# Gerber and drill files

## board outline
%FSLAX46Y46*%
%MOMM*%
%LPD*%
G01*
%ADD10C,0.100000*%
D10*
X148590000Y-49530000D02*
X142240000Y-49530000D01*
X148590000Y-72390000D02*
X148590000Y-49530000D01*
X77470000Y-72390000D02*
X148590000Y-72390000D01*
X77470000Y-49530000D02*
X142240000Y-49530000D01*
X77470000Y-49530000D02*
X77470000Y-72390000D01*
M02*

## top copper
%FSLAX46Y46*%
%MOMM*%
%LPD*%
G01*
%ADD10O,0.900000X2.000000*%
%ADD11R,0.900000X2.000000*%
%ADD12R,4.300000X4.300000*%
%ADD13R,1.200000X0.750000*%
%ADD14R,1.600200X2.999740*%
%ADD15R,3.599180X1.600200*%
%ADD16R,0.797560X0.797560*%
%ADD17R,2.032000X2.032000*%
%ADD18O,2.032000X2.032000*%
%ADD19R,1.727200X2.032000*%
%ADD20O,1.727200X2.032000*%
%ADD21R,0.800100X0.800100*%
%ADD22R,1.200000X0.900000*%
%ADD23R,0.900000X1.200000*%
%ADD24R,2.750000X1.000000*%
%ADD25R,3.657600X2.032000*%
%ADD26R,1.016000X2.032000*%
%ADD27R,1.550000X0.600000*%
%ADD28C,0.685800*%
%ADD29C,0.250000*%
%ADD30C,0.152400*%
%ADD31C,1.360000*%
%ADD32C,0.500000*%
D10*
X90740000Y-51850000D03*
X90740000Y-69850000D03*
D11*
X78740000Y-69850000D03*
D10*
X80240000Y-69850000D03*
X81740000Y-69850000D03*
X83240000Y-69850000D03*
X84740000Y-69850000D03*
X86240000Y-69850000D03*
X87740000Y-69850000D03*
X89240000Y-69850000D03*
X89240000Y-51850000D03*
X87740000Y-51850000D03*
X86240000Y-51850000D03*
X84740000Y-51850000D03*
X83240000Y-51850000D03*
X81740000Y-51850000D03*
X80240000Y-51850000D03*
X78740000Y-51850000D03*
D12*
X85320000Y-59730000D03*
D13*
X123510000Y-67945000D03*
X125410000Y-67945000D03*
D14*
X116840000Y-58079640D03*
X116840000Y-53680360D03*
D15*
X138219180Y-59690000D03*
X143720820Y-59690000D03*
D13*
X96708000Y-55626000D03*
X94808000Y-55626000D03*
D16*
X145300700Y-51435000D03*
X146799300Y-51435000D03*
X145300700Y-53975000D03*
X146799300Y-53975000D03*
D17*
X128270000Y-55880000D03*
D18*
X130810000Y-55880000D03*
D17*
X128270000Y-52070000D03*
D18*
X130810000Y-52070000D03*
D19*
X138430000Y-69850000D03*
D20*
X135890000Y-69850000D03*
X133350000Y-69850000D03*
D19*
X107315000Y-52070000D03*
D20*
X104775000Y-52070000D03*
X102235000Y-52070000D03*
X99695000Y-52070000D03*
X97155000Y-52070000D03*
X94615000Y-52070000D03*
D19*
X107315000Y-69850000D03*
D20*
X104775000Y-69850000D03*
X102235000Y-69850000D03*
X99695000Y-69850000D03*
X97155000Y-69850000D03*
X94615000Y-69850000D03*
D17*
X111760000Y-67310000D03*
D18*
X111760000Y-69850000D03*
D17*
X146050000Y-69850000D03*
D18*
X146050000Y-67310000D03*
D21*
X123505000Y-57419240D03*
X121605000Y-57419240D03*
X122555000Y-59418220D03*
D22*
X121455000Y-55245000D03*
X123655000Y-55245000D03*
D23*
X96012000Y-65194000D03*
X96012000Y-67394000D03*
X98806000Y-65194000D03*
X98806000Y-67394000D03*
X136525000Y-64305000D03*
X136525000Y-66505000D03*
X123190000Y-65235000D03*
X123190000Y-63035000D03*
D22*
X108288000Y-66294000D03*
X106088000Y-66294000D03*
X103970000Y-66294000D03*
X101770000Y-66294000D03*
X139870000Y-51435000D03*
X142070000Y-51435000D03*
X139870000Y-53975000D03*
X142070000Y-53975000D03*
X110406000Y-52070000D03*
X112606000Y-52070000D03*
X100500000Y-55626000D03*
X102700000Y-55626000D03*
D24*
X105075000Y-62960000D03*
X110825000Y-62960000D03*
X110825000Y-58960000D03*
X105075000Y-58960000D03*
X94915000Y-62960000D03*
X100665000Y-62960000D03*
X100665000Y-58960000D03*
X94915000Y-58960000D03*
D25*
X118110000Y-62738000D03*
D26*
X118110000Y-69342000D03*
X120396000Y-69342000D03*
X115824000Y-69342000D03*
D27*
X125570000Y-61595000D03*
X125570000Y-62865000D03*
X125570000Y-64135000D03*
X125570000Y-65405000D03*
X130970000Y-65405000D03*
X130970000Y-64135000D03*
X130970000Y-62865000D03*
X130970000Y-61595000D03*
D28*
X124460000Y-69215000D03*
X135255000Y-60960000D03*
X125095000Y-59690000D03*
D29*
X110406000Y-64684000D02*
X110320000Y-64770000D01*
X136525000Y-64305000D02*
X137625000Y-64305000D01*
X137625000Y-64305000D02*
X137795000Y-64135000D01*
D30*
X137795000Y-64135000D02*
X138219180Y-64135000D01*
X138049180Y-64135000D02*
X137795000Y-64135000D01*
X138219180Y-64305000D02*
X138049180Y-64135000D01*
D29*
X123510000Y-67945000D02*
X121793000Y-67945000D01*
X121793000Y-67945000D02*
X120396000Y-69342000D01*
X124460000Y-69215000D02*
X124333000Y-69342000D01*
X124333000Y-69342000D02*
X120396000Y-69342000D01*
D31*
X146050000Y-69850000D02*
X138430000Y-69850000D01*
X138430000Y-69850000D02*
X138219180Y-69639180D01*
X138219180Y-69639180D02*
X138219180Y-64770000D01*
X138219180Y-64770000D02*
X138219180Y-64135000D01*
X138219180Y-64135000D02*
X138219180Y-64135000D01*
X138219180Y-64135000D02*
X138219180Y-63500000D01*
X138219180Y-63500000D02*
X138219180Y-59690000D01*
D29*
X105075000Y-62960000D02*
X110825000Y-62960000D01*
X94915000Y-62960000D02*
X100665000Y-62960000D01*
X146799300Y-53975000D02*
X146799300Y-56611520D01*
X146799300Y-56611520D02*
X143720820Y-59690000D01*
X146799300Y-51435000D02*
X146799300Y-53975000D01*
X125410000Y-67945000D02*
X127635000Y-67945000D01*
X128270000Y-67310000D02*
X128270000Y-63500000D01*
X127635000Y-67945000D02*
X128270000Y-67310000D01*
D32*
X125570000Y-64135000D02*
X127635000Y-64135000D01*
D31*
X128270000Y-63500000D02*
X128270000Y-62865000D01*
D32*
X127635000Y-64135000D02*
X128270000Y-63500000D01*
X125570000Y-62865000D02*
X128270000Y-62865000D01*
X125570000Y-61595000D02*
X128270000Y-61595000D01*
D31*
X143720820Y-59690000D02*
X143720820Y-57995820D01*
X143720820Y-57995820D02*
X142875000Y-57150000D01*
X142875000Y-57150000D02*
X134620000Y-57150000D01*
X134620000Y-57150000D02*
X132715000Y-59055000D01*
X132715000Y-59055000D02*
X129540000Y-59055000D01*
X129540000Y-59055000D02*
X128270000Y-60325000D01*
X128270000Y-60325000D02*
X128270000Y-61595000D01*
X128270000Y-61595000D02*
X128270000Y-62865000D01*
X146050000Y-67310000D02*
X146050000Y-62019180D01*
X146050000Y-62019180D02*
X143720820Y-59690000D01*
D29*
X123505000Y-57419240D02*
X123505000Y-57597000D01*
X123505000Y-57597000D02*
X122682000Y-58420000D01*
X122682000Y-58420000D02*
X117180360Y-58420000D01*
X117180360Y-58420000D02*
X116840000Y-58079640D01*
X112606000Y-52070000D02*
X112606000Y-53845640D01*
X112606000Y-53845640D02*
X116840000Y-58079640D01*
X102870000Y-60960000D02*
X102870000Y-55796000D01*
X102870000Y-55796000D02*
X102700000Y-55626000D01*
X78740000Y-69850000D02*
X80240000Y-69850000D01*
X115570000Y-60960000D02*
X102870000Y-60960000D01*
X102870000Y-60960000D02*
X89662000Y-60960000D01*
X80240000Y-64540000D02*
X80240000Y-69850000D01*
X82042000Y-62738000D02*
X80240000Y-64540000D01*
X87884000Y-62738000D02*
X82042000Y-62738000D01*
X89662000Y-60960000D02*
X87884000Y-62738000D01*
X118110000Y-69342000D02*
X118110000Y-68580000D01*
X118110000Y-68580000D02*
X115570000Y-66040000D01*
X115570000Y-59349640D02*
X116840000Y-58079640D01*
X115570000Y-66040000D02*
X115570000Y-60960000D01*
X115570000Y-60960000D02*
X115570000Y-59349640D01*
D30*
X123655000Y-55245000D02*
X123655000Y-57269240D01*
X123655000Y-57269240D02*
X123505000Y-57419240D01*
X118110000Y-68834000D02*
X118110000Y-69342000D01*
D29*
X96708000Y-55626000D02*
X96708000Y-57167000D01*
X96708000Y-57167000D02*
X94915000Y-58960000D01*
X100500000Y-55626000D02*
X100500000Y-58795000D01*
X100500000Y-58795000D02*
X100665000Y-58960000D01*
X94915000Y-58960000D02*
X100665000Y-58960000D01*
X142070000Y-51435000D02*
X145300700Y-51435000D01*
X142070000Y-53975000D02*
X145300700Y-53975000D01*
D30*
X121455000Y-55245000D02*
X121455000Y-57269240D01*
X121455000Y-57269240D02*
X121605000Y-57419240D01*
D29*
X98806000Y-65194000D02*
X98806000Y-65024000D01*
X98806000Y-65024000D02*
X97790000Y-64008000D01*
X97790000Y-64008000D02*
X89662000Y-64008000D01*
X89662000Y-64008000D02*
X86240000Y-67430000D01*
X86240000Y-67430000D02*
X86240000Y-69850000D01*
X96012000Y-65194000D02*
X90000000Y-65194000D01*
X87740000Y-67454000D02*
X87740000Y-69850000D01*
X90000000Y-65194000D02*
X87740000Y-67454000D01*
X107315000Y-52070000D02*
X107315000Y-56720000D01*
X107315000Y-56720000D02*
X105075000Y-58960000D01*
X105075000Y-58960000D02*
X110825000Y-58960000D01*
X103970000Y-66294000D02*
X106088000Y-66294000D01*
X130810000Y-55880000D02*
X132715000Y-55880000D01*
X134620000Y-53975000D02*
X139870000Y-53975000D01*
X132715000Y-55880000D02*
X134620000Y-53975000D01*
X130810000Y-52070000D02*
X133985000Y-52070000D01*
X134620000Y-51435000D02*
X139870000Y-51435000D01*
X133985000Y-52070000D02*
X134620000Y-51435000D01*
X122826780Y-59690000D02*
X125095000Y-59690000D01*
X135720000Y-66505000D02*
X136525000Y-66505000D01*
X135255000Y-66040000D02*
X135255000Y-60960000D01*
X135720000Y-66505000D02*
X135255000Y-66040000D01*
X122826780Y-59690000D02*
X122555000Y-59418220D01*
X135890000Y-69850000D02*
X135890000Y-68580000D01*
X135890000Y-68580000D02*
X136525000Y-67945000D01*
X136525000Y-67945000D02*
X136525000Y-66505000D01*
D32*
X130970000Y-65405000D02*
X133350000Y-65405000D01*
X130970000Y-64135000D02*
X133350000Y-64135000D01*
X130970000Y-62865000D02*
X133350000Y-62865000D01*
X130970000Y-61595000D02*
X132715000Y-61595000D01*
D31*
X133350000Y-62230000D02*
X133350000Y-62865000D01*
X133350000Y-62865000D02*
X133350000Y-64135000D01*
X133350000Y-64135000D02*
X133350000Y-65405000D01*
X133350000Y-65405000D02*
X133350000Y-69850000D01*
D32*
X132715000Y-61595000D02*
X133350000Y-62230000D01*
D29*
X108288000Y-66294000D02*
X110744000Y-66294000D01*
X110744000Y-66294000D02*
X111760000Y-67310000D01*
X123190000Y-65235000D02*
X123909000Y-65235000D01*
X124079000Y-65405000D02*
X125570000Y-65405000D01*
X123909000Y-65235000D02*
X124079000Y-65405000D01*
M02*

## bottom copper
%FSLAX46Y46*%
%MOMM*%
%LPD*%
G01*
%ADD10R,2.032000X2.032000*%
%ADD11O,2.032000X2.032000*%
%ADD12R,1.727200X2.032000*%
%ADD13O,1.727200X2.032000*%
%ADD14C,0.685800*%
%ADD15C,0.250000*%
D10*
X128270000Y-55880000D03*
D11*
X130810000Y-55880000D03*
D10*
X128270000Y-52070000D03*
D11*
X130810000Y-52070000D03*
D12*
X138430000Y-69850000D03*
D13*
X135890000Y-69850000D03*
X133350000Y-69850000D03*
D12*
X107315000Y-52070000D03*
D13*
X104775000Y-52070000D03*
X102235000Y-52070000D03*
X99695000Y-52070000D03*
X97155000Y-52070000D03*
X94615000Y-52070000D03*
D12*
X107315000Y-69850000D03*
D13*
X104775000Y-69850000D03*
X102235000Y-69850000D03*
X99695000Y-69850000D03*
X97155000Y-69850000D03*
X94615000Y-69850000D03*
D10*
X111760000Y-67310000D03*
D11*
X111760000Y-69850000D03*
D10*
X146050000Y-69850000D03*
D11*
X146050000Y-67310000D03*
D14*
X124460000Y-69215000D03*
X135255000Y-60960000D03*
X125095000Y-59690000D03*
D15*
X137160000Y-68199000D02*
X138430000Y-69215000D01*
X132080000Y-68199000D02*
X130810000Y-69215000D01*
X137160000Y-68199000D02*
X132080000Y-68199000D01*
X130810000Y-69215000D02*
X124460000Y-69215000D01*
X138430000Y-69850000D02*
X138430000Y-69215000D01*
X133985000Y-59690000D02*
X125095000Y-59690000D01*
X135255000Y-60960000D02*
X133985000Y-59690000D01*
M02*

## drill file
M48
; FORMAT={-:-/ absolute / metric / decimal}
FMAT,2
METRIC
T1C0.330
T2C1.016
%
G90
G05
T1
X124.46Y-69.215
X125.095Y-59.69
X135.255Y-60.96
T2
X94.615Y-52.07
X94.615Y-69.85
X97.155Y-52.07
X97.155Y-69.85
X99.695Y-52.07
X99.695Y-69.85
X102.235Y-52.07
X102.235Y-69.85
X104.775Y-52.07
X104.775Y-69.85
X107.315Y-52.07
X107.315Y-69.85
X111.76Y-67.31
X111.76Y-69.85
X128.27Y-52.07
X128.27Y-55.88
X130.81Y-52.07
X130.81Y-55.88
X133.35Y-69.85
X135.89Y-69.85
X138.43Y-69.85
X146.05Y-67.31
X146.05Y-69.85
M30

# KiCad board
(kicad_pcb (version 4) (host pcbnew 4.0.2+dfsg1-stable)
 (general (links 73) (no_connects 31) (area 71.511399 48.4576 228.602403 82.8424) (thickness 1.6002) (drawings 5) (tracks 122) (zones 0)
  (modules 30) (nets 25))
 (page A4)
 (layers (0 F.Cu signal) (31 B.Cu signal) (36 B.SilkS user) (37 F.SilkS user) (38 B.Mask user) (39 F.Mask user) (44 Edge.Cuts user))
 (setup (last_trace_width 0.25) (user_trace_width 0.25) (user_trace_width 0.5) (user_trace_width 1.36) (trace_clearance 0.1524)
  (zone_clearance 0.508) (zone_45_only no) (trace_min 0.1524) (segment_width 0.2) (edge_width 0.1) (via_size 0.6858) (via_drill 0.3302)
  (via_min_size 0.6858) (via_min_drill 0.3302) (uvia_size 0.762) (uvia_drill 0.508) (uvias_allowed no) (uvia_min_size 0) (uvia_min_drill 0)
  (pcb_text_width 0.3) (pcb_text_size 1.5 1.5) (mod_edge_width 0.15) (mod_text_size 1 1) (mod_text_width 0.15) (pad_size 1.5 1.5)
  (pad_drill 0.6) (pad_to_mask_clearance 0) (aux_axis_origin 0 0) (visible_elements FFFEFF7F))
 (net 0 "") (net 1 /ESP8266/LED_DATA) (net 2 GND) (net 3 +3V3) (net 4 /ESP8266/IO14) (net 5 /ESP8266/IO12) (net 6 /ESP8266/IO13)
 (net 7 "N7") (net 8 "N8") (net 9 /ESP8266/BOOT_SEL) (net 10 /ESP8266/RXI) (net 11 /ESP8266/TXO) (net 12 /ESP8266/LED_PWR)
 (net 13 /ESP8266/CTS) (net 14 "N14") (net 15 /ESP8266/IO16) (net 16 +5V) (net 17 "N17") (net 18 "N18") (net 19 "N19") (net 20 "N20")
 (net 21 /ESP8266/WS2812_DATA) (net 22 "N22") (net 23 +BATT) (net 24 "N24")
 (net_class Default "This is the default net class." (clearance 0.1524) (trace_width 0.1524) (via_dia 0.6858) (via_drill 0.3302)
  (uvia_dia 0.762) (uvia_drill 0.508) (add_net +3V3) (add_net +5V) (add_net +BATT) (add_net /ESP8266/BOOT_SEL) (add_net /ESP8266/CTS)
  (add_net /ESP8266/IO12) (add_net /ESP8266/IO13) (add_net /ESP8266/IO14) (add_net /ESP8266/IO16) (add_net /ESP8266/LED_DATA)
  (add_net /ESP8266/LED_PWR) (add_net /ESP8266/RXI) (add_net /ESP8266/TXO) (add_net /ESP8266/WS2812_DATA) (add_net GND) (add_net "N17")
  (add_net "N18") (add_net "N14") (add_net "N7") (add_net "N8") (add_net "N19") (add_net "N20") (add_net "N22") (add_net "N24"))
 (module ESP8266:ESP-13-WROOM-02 (layer F.Cu) (at 78.74 69.85 90)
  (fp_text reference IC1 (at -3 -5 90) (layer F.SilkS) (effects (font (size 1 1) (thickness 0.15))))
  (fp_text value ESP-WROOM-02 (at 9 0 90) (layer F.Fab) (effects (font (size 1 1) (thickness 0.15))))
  (pad 10 smd oval (at 18 12 90) (size 2 0.9) (layers F.Cu F.Mask) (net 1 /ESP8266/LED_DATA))
  (pad 9 smd oval (at 0 12 90) (size 2 0.9) (layers F.Cu F.Mask) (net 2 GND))
  (pad 1 smd rect (at 0 0 90) (size 2 0.9) (layers F.Cu F.Mask) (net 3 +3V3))
  (pad 2 smd oval (at 0 1.5 90) (size 2 0.9) (layers F.Cu F.Mask) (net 3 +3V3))
  (pad 3 smd oval (at 0 3 90) (size 2 0.9) (layers F.Cu F.Mask) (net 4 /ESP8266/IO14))
  (pad 4 smd oval (at 0 4.5 90) (size 2 0.9) (layers F.Cu F.Mask) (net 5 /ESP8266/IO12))
  (pad 5 smd oval (at 0 6 90) (size 2 0.9) (layers F.Cu F.Mask) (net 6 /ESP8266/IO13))
  (pad 6 smd oval (at 0 7.5 90) (size 2 0.9) (layers F.Cu F.Mask) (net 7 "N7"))
  (pad 7 smd oval (at 0 9 90) (size 2 0.9) (layers F.Cu F.Mask) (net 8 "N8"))
  (pad 8 smd oval (at 0 10.5 90) (size 2 0.9) (layers F.Cu F.Mask) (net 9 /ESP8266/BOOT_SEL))
  (pad 11 smd oval (at 18 10.5 90) (size 2 0.9) (layers F.Cu F.Mask) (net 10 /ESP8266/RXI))
  (pad 12 smd oval (at 18 9 90) (size 2 0.9) (layers F.Cu F.Mask) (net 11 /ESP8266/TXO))
  (pad 13 smd oval (at 18 7.5 90) (size 2 0.9) (layers F.Cu F.Mask) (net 2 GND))
  (pad 14 smd oval (at 18 6 90) (size 2 0.9) (layers F.Cu F.Mask) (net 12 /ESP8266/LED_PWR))
  (pad 15 smd oval (at 18 4.5 90) (size 2 0.9) (layers F.Cu F.Mask) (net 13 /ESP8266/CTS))
  (pad 16 smd oval (at 18 3 90) (size 2 0.9) (layers F.Cu F.Mask) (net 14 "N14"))
  (pad 17 smd oval (at 18 1.5 90) (size 2 0.9) (layers F.Cu F.Mask) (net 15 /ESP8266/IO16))
  (pad 18 smd oval (at 18 0 90) (size 2 0.9) (layers F.Cu F.Mask) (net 2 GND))
  (pad PAD smd rect (at 10.12 6.58 90) (size 4.3 4.3) (layers F.Cu F.Mask)))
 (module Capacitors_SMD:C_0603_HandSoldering (layer F.Cu) (at 124.46 67.945)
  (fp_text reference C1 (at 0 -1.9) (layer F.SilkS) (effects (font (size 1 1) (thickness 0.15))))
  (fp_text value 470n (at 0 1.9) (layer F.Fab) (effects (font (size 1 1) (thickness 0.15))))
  (pad 1 smd rect (at -0.95 0) (size 1.2 0.75) (layers F.Cu F.Mask) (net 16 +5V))
  (pad 2 smd rect (at 0.95 0) (size 1.2 0.75) (layers F.Cu F.Mask) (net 2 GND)))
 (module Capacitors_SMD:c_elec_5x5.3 (layer F.Cu) (at 116.84 55.88 270)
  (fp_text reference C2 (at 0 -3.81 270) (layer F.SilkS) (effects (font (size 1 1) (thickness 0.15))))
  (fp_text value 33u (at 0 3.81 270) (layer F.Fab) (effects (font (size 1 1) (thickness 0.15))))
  (pad 1 smd rect (at 2.19964 0 270) (size 2.99974 1.6002) (layers F.Cu F.Mask) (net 3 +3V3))
  (pad 2 smd rect (at -2.19964 0 270) (size 2.99974 1.6002) (layers F.Cu F.Mask) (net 2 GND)))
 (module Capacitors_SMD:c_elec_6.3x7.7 (layer F.Cu) (at 140.97 59.69 180)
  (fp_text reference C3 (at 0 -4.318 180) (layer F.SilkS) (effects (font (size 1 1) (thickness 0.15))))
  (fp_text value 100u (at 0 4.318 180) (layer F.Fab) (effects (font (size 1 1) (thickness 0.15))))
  (pad 1 smd rect (at 2.75082 0 180) (size 3.59918 1.6002) (layers F.Cu F.Mask) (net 16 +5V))
  (pad 2 smd rect (at -2.75082 0 180) (size 3.59918 1.6002) (layers F.Cu F.Mask) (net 2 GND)))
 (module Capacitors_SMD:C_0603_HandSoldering (layer F.Cu) (at 95.758 55.626 180)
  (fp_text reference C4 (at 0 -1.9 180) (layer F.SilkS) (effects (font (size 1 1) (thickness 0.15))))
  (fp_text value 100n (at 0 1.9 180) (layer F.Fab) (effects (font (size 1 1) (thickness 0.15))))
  (pad 1 smd rect (at -0.95 0 180) (size 1.2 0.75) (layers F.Cu F.Mask) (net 13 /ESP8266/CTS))
  (pad 2 smd rect (at 0.95 0 180) (size 1.2 0.75) (layers F.Cu F.Mask) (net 2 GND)))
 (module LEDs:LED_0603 (layer F.Cu) (at 146.05 51.435 180)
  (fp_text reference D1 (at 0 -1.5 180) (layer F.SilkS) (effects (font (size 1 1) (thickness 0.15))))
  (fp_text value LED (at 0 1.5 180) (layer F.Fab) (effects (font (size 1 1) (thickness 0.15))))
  (pad 2 smd rect (at 0.7493 0) (size 0.79756 0.79756) (layers F.Cu F.Mask) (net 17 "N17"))
  (pad 1 smd rect (at -0.7493 0) (size 0.79756 0.79756) (layers F.Cu F.Mask) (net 2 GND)))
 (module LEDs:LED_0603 (layer F.Cu) (at 146.05 53.975 180)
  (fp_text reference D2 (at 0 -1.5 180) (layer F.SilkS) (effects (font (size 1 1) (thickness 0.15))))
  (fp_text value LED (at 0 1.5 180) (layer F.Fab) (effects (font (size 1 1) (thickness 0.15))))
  (pad 2 smd rect (at 0.7493 0) (size 0.79756 0.79756) (layers F.Cu F.Mask) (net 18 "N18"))
  (pad 1 smd rect (at -0.7493 0) (size 0.79756 0.79756) (layers F.Cu F.Mask) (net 2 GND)))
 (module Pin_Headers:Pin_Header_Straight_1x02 (layer F.Cu) (at 128.27 55.88 90)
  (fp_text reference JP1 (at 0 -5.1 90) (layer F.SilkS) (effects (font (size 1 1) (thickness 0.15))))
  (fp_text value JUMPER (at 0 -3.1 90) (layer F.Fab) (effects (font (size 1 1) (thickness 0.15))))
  (pad 1 thru_hole rect (at 0 0 90) (size 2.032 2.032) (drill 1.016) (layers *.Cu *.Mask F.SilkS) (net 6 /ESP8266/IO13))
  (pad 2 thru_hole oval (at 0 2.54 90) (size 2.032 2.032) (drill 1.016) (layers *.Cu *.Mask F.SilkS) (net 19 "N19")))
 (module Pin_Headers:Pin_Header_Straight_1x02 (layer F.Cu) (at 128.27 52.07 90)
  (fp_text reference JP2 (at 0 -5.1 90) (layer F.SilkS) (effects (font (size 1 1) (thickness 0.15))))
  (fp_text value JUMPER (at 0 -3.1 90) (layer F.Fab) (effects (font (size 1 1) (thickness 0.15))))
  (pad 1 thru_hole rect (at 0 0 90) (size 2.032 2.032) (drill 1.016) (layers *.Cu *.Mask F.SilkS) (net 5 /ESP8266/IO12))
  (pad 2 thru_hole oval (at 0 2.54 90) (size 2.032 2.032) (drill 1.016) (layers *.Cu *.Mask F.SilkS) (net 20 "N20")))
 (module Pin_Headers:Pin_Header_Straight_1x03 (layer F.Cu) (at 138.43 69.85 270)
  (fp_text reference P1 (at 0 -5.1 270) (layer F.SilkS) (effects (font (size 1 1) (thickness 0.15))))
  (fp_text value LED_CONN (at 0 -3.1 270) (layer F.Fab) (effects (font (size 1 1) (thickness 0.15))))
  (pad 1 thru_hole rect (at 0 0 270) (size 2.032 1.7272) (drill 1.016) (layers *.Cu *.Mask F.SilkS) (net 16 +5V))
  (pad 2 thru_hole oval (at 0 2.54 270) (size 2.032 1.7272) (drill 1.016) (layers *.Cu *.Mask F.SilkS) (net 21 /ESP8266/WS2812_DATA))
  (pad 3 thru_hole oval (at 0 5.08 270) (size 2.032 1.7272) (drill 1.016) (layers *.Cu *.Mask F.SilkS) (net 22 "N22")))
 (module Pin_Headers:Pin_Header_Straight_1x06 (layer F.Cu) (at 107.315 52.07 270)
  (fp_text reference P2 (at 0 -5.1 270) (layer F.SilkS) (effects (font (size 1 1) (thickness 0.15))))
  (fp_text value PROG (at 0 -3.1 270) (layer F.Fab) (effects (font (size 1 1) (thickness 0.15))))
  (pad 1 thru_hole rect (at 0 0 270) (size 2.032 1.7272) (drill 1.016) (layers *.Cu *.Mask F.SilkS) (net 9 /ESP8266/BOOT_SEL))
  (pad 2 thru_hole oval (at 0 2.54 270) (size 2.032 1.7272) (drill 1.016) (layers *.Cu *.Mask F.SilkS) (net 10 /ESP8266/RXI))
  (pad 3 thru_hole oval (at 0 5.08 270) (size 2.032 1.7272) (drill 1.016) (layers *.Cu *.Mask F.SilkS) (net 11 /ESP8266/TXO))
  (pad 4 thru_hole oval (at 0 7.62 270) (size 2.032 1.7272) (drill 1.016) (layers *.Cu *.Mask F.SilkS) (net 16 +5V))
  (pad 5 thru_hole oval (at 0 10.16 270) (size 2.032 1.7272) (drill 1.016) (layers *.Cu *.Mask F.SilkS) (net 13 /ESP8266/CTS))
  (pad 6 thru_hole oval (at 0 12.7 270) (size 2.032 1.7272) (drill 1.016) (layers *.Cu *.Mask F.SilkS) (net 2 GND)))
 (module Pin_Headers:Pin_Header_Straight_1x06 (layer F.Cu) (at 107.315 69.85 270)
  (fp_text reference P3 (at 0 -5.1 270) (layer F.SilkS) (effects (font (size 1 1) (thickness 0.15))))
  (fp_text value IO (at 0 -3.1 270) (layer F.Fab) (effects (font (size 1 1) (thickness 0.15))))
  (pad 1 thru_hole rect (at 0 0 270) (size 2.032 1.7272) (drill 1.016) (layers *.Cu *.Mask F.SilkS) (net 3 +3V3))
  (pad 2 thru_hole oval (at 0 2.54 270) (size 2.032 1.7272) (drill 1.016) (layers *.Cu *.Mask F.SilkS) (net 5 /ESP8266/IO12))
  (pad 3 thru_hole oval (at 0 5.08 270) (size 2.032 1.7272) (drill 1.016) (layers *.Cu *.Mask F.SilkS) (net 6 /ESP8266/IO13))
  (pad 4 thru_hole oval (at 0 7.62 270) (size 2.032 1.7272) (drill 1.016) (layers *.Cu *.Mask F.SilkS) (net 4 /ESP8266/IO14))
  (pad 5 thru_hole oval (at 0 10.16 270) (size 2.032 1.7272) (drill 1.016) (layers *.Cu *.Mask F.SilkS) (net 15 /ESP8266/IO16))
  (pad 6 thru_hole oval (at 0 12.7 270) (size 2.032 1.7272) (drill 1.016) (layers *.Cu *.Mask F.SilkS) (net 2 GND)))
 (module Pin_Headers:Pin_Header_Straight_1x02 (layer F.Cu) (at 111.76 67.31)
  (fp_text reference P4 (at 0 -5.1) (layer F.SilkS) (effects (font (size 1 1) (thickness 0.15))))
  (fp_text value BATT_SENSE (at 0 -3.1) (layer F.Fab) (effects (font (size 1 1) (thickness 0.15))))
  (pad 1 thru_hole rect (at 0 0) (size 2.032 2.032) (drill 1.016) (layers *.Cu *.Mask F.SilkS) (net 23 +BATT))
  (pad 2 thru_hole oval (at 0 2.54) (size 2.032 2.032) (drill 1.016) (layers *.Cu *.Mask F.SilkS) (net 2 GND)))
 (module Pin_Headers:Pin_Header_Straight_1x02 (layer F.Cu) (at 146.05 69.85 180)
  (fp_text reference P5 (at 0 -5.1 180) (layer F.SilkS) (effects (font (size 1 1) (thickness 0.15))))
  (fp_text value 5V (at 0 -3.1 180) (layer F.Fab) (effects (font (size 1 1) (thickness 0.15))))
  (pad 1 thru_hole rect (at 0 0 180) (size 2.032 2.032) (drill 1.016) (layers *.Cu *.Mask F.SilkS) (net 16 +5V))
  (pad 2 thru_hole oval (at 0 2.54 180) (size 2.032 2.032) (drill 1.016) (layers *.Cu *.Mask F.SilkS) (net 2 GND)))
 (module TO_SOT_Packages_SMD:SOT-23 (layer F.Cu) (at 122.555 58.42 180)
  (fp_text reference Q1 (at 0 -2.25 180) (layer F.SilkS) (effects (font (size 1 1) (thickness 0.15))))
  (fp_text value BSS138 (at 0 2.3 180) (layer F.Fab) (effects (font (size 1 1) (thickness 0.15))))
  (pad 1 smd rect (at -0.95 1.00076 180) (size 0.8001 0.8001) (layers F.Cu F.Mask) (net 3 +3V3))
  (pad 2 smd rect (at 0.95 1.00076 180) (size 0.8001 0.8001) (layers F.Cu F.Mask) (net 1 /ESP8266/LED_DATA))
  (pad 3 smd rect (at 0 -0.99822 180) (size 0.8001 0.8001) (layers F.Cu F.Mask) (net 21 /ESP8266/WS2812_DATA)))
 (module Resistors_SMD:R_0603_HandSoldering (layer F.Cu) (at 122.555 55.245)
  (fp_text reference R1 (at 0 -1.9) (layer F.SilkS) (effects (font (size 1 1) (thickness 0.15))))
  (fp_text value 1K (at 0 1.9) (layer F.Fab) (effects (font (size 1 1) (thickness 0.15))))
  (pad 1 smd rect (at -1.1 0) (size 1.2 0.9) (layers F.Cu F.Mask) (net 1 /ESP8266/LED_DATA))
  (pad 2 smd rect (at 1.1 0) (size 1.2 0.9) (layers F.Cu F.Mask) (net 3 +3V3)))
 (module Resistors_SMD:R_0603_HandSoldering (layer F.Cu) (at 96.012 66.294 270)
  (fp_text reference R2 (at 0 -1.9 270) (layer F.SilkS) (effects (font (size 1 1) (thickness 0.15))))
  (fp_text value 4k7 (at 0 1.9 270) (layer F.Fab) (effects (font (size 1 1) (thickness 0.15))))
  (pad 1 smd rect (at -1.1 0 270) (size 1.2 0.9) (layers F.Cu F.Mask) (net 8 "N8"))
  (pad 2 smd rect (at 1.1 0 270) (size 1.2 0.9) (layers F.Cu F.Mask) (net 3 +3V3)))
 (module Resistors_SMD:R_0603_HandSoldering (layer F.Cu) (at 98.806 66.294 270)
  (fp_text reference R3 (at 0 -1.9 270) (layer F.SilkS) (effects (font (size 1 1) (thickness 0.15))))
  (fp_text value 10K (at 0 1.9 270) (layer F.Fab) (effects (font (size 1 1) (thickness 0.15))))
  (pad 1 smd rect (at -1.1 0 270) (size 1.2 0.9) (layers F.Cu F.Mask) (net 7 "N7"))
  (pad 2 smd rect (at 1.1 0 270) (size 1.2 0.9) (layers F.Cu F.Mask) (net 2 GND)))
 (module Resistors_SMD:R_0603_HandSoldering (layer F.Cu) (at 136.525 65.405 270)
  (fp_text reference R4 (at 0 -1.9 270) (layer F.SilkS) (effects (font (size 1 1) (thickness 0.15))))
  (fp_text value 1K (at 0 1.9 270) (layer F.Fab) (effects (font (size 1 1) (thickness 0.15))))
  (pad 1 smd rect (at -1.1 0 270) (size 1.2 0.9) (layers F.Cu F.Mask) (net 16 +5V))
  (pad 2 smd rect (at 1.1 0 270) (size 1.2 0.9) (layers F.Cu F.Mask) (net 21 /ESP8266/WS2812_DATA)))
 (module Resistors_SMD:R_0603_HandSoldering (layer F.Cu) (at 123.19 64.135 90)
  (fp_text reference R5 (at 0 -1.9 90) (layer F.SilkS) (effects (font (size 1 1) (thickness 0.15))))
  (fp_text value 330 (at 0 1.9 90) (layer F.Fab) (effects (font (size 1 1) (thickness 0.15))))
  (pad 1 smd rect (at -1.1 0 90) (size 1.2 0.9) (layers F.Cu F.Mask) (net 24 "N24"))
  (pad 2 smd rect (at 1.1 0 90) (size 1.2 0.9) (layers F.Cu F.Mask) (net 12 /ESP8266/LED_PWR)))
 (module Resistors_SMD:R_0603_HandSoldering (layer F.Cu) (at 107.188 66.294 180)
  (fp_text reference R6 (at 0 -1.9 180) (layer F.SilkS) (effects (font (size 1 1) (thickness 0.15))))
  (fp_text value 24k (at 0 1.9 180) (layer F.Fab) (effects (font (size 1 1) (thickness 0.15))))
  (pad 1 smd rect (at -1.1 0 180) (size 1.2 0.9) (layers F.Cu F.Mask) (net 23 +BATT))
  (pad 2 smd rect (at 1.1 0 180) (size 1.2 0.9) (layers F.Cu F.Mask) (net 14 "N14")))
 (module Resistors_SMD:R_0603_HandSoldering (layer F.Cu) (at 102.87 66.294 180)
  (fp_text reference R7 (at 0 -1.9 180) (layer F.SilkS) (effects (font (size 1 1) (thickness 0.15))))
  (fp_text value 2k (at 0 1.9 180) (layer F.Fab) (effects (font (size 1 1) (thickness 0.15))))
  (pad 1 smd rect (at -1.1 0 180) (size 1.2 0.9) (layers F.Cu F.Mask) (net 14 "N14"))
  (pad 2 smd rect (at 1.1 0 180) (size 1.2 0.9) (layers F.Cu F.Mask) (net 2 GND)))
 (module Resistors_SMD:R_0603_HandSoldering (layer F.Cu) (at 140.97 51.435)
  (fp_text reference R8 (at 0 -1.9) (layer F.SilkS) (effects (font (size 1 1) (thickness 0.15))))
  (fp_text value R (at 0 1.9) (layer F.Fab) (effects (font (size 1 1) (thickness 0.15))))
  (pad 1 smd rect (at -1.1 0) (size 1.2 0.9) (layers F.Cu F.Mask) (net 20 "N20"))
  (pad 2 smd rect (at 1.1 0) (size 1.2 0.9) (layers F.Cu F.Mask) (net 17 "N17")))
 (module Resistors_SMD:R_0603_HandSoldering (layer F.Cu) (at 140.97 53.975)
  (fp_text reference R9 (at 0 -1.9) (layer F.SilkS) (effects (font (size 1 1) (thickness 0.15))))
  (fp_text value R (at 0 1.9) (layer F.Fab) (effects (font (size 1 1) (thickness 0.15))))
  (pad 1 smd rect (at -1.1 0) (size 1.2 0.9) (layers F.Cu F.Mask) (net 19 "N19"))
  (pad 2 smd rect (at 1.1 0) (size 1.2 0.9) (layers F.Cu F.Mask) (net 18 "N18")))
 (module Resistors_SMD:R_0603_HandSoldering (layer F.Cu) (at 111.506 52.07)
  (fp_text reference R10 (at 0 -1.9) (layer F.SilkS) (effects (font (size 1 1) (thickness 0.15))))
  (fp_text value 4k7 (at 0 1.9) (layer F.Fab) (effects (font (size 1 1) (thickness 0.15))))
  (pad 1 smd rect (at -1.1 0) (size 1.2 0.9) (layers F.Cu F.Mask) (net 9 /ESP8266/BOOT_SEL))
  (pad 2 smd rect (at 1.1 0) (size 1.2 0.9) (layers F.Cu F.Mask) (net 3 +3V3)))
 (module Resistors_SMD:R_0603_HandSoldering (layer F.Cu) (at 101.6 55.626)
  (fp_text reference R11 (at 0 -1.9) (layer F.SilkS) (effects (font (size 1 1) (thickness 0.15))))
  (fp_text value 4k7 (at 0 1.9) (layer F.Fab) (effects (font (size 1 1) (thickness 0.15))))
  (pad 1 smd rect (at -1.1 0) (size 1.2 0.9) (layers F.Cu F.Mask) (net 13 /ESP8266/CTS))
  (pad 2 smd rect (at 1.1 0) (size 1.2 0.9) (layers F.Cu F.Mask) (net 3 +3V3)))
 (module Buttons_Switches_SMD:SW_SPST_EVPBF (layer F.Cu) (at 107.95 60.96 180)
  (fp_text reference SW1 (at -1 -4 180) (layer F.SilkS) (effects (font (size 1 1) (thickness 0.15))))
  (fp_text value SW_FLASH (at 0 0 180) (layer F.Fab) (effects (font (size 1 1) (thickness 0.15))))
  (pad 1 smd rect (at 2.875 -2 180) (size 2.75 1) (layers F.Cu F.Mask) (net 2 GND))
  (pad 1 smd rect (at -2.875 -2 180) (size 2.75 1) (layers F.Cu F.Mask) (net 2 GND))
  (pad 2 smd rect (at -2.875 2 180) (size 2.75 1) (layers F.Cu F.Mask) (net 9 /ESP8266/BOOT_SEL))
  (pad 2 smd rect (at 2.875 2 180) (size 2.75 1) (layers F.Cu F.Mask) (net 9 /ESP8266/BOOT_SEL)))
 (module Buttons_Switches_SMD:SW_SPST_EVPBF (layer F.Cu) (at 97.79 60.96 180)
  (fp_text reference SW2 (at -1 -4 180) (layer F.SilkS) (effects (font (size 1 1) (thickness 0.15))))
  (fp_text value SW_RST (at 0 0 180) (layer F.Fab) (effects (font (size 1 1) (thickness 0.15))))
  (pad 1 smd rect (at 2.875 -2 180) (size 2.75 1) (layers F.Cu F.Mask) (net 2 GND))
  (pad 1 smd rect (at -2.875 -2 180) (size 2.75 1) (layers F.Cu F.Mask) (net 2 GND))
  (pad 2 smd rect (at -2.875 2 180) (size 2.75 1) (layers F.Cu F.Mask) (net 13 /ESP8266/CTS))
  (pad 2 smd rect (at 2.875 2 180) (size 2.75 1) (layers F.Cu F.Mask) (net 13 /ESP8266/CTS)))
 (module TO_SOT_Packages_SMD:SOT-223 (layer F.Cu) (at 118.11 66.04)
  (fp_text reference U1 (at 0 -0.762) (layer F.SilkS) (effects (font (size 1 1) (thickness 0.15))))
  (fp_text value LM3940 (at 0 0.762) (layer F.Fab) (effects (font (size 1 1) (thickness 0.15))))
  (pad 4 smd rect (at 0 -3.302) (size 3.6576 2.032) (layers F.Cu F.Mask))
  (pad 2 smd rect (at 0 3.302) (size 1.016 2.032) (layers F.Cu F.Mask) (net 3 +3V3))
  (pad 3 smd rect (at 2.286 3.302) (size 1.016 2.032) (layers F.Cu F.Mask) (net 16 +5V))
  (pad 1 smd rect (at -2.286 3.302) (size 1.016 2.032) (layers F.Cu F.Mask) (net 2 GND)))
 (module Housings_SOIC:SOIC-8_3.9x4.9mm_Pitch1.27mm (layer F.Cu) (at 128.27 63.5)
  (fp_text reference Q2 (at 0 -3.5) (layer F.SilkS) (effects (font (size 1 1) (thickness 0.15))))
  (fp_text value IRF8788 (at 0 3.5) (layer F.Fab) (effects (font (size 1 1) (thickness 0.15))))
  (pad 1 smd rect (at -2.7 -1.905) (size 1.55 0.6) (layers F.Cu F.Mask) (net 2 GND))
  (pad 2 smd rect (at -2.7 -0.635) (size 1.55 0.6) (layers F.Cu F.Mask) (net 2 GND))
  (pad 3 smd rect (at -2.7 0.635) (size 1.55 0.6) (layers F.Cu F.Mask) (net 2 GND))
  (pad 4 smd rect (at -2.7 1.905) (size 1.55 0.6) (layers F.Cu F.Mask) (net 24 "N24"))
  (pad 5 smd rect (at 2.7 1.905) (size 1.55 0.6) (layers F.Cu F.Mask) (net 22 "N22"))
  (pad 6 smd rect (at 2.7 0.635) (size 1.55 0.6) (layers F.Cu F.Mask) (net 22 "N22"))
  (pad 7 smd rect (at 2.7 -0.635) (size 1.55 0.6) (layers F.Cu F.Mask) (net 22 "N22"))
  (pad 8 smd rect (at 2.7 -1.905) (size 1.55 0.6) (layers F.Cu F.Mask) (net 22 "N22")))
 (gr_line (start 148.59 49.53) (end 142.24 49.53) (angle 90) (layer Edge.Cuts) (width 0.1))
 (gr_line (start 148.59 72.39) (end 148.59 49.53) (angle 90) (layer Edge.Cuts) (width 0.1))
 (gr_line (start 77.47 72.39) (end 148.59 72.39) (angle 90) (layer Edge.Cuts) (width 0.1))
 (gr_line (start 77.47 49.53) (end 142.24 49.53) (angle 90) (layer Edge.Cuts) (width 0.1))
 (gr_line (start 77.47 49.53) (end 77.47 72.39) (angle 90) (layer Edge.Cuts) (width 0.1))
 (segment (start 110.406 64.684) (end 110.32 64.77) (width 0.25) (layer F.Cu) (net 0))
 (segment (start 136.525 64.305) (end 137.625 64.305) (width 0.25) (layer F.Cu) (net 16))
 (segment (start 137.625 64.305) (end 137.795 64.135) (width 0.25) (layer F.Cu) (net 16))
 (segment (start 137.795 64.135) (end 138.21918 64.135) (width 0.1524) (layer F.Cu) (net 16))
 (segment (start 138.04918 64.135) (end 137.795 64.135) (width 0.1524) (layer F.Cu) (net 16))
 (segment (start 138.21918 64.305) (end 138.04918 64.135) (width 0.1524) (layer F.Cu) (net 16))
 (segment (start 123.51 67.945) (end 121.793 67.945) (width 0.25) (layer F.Cu) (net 16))
 (segment (start 121.793 67.945) (end 120.396 69.342) (width 0.25) (layer F.Cu) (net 16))
 (via (at 124.46 69.215) (size 0.6858) (drill 0.3302) (layers F.Cu B.Cu) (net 16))
 (segment (start 124.46 69.215) (end 124.333 69.342) (width 0.25) (layer F.Cu) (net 16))
 (segment (start 124.333 69.342) (end 120.396 69.342) (width 0.25) (layer F.Cu) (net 16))
 (segment (start 137.16 68.199) (end 138.43 69.215) (width 0.25) (layer B.Cu) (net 16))
 (segment (start 132.08 68.199) (end 130.81 69.215) (width 0.25) (layer B.Cu) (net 16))
 (segment (start 137.16 68.199) (end 132.08 68.199) (width 0.25) (layer B.Cu) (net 16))
 (segment (start 130.81 69.215) (end 124.46 69.215) (width 0.25) (layer B.Cu) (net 16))
 (segment (start 138.43 69.85) (end 138.43 69.215) (width 0.25) (layer B.Cu) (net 16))
 (segment (start 146.05 69.85) (end 138.43 69.85) (width 1.36) (layer F.Cu) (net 16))
 (segment (start 138.43 69.85) (end 138.21918 69.63918) (width 1.36) (layer F.Cu) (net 16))
 (segment (start 138.21918 69.63918) (end 138.21918 64.77) (width 1.36) (layer F.Cu) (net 16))
 (segment (start 138.21918 64.77) (end 138.21918 64.135) (width 1.36) (layer F.Cu) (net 16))
 (segment (start 138.21918 64.135) (end 138.21918 64.135) (width 1.36) (layer F.Cu) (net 16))
 (segment (start 138.21918 64.135) (end 138.21918 63.5) (width 1.36) (layer F.Cu) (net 16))
 (segment (start 138.21918 63.5) (end 138.21918 59.69) (width 1.36) (layer F.Cu) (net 16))
 (segment (start 105.075 62.96) (end 110.825 62.96) (width 0.25) (layer F.Cu) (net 2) (status 30))
 (segment (start 94.915 62.96) (end 100.665 62.96) (width 0.25) (layer F.Cu) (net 2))
 (segment (start 146.7993 53.975) (end 146.7993 56.61152) (width 0.25) (layer F.Cu) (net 2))
 (segment (start 146.7993 56.61152) (end 143.72082 59.69) (width 0.25) (layer F.Cu) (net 2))
 (segment (start 146.7993 51.435) (end 146.7993 53.975) (width 0.25) (layer F.Cu) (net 2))
 (segment (start 125.41 67.945) (end 127.635 67.945) (width 0.25) (layer F.Cu) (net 2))
 (segment (start 128.27 67.31) (end 128.27 63.5) (width 0.25) (layer F.Cu) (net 2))
 (segment (start 127.635 67.945) (end 128.27 67.31) (width 0.25) (layer F.Cu) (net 2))
 (segment (start 125.57 64.135) (end 127.635 64.135) (width 0.5) (layer F.Cu) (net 2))
 (segment (start 128.27 63.5) (end 128.27 62.865) (width 1.36) (layer F.Cu) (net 2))
 (segment (start 127.635 64.135) (end 128.27 63.5) (width 0.5) (layer F.Cu) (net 2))
 (segment (start 125.57 62.865) (end 128.27 62.865) (width 0.5) (layer F.Cu) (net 2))
 (segment (start 125.57 61.595) (end 128.27 61.595) (width 0.5) (layer F.Cu) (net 2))
 (segment (start 143.72082 59.69) (end 143.72082 57.99582) (width 1.36) (layer F.Cu) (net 2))
 (segment (start 143.72082 57.99582) (end 142.875 57.15) (width 1.36) (layer F.Cu) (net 2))
 (segment (start 142.875 57.15) (end 134.62 57.15) (width 1.36) (layer F.Cu) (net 2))
 (segment (start 134.62 57.15) (end 132.715 59.055) (width 1.36) (layer F.Cu) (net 2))
 (segment (start 132.715 59.055) (end 129.54 59.055) (width 1.36) (layer F.Cu) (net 2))
 (segment (start 129.54 59.055) (end 128.27 60.325) (width 1.36) (layer F.Cu) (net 2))
 (segment (start 128.27 60.325) (end 128.27 61.595) (width 1.36) (layer F.Cu) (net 2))
 (segment (start 128.27 61.595) (end 128.27 62.865) (width 1.36) (layer F.Cu) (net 2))
 (segment (start 146.05 67.31) (end 146.05 62.01918) (width 1.36) (layer F.Cu) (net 2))
 (segment (start 146.05 62.01918) (end 143.72082 59.69) (width 1.36) (layer F.Cu) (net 2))
 (segment (start 123.505 57.41924) (end 123.505 57.597) (width 0.25) (layer F.Cu) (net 3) (status C00000))
 (segment (start 123.505 57.597) (end 122.682 58.42) (width 0.25) (layer F.Cu) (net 3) (status 400000))
 (segment (start 122.682 58.42) (end 117.18036 58.42) (width 0.25) (layer F.Cu) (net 3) (status 800000))
 (segment (start 117.18036 58.42) (end 116.84 58.07964) (width 0.25) (layer F.Cu) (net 3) (status C00000))
 (segment (start 112.606 52.07) (end 112.606 53.84564) (width 0.25) (layer F.Cu) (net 3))
 (segment (start 112.606 53.84564) (end 116.84 58.07964) (width 0.25) (layer F.Cu) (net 3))
 (segment (start 102.87 60.96) (end 102.87 55.796) (width 0.25) (layer F.Cu) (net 3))
 (segment (start 102.87 55.796) (end 102.7 55.626) (width 0.25) (layer F.Cu) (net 3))
 (segment (start 78.74 69.85) (end 80.24 69.85) (width 0.25) (layer F.Cu) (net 3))
 (segment (start 115.57 60.96) (end 102.87 60.96) (width 0.25) (layer F.Cu) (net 3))
 (segment (start 102.87 60.96) (end 89.662 60.96) (width 0.25) (layer F.Cu) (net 3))
 (segment (start 80.24 64.54) (end 80.24 69.85) (width 0.25) (layer F.Cu) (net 3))
 (segment (start 82.042 62.738) (end 80.24 64.54) (width 0.25) (layer F.Cu) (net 3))
 (segment (start 87.884 62.738) (end 82.042 62.738) (width 0.25) (layer F.Cu) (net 3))
 (segment (start 89.662 60.96) (end 87.884 62.738) (width 0.25) (layer F.Cu) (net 3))
 (segment (start 118.11 69.342) (end 118.11 68.58) (width 0.25) (layer F.Cu) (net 3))
 (segment (start 118.11 68.58) (end 115.57 66.04) (width 0.25) (layer F.Cu) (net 3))
 (segment (start 115.57 59.34964) (end 116.84 58.07964) (width 0.25) (layer F.Cu) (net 3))
 (segment (start 115.57 66.04) (end 115.57 60.96) (width 0.25) (layer F.Cu) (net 3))
 (segment (start 115.57 60.96) (end 115.57 59.34964) (width 0.25) (layer F.Cu) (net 3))
 (segment (start 123.655 55.245) (end 123.655 57.26924) (width 0.1524) (layer F.Cu) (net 3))
 (segment (start 123.655 57.26924) (end 123.505 57.41924) (width 0.1524) (layer F.Cu) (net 3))
 (segment (start 118.11 68.834) (end 118.11 69.342) (width 0.1524) (layer F.Cu) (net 3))
 (segment (start 96.708 55.626) (end 96.708 57.167) (width 0.25) (layer F.Cu) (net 13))
 (segment (start 96.708 57.167) (end 94.915 58.96) (width 0.25) (layer F.Cu) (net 13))
 (segment (start 100.5 55.626) (end 100.5 58.795) (width 0.25) (layer F.Cu) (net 13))
 (segment (start 100.5 58.795) (end 100.665 58.96) (width 0.25) (layer F.Cu) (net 13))
 (segment (start 94.915 58.96) (end 100.665 58.96) (width 0.25) (layer F.Cu) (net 13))
 (segment (start 142.07 51.435) (end 145.3007 51.435) (width 0.25) (layer F.Cu) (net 17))
 (segment (start 142.07 53.975) (end 145.3007 53.975) (width 0.25) (layer F.Cu) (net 18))
 (segment (start 121.455 55.245) (end 121.455 57.26924) (width 0.1524) (layer F.Cu) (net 1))
 (segment (start 121.455 57.26924) (end 121.605 57.41924) (width 0.1524) (layer F.Cu) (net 1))
 (segment (start 98.806 65.194) (end 98.806 65.024) (width 0.25) (layer F.Cu) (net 7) (status C00000))
 (segment (start 98.806 65.024) (end 97.79 64.008) (width 0.25) (layer F.Cu) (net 7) (status 400000))
 (segment (start 97.79 64.008) (end 89.662 64.008) (width 0.25) (layer F.Cu) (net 7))
 (segment (start 89.662 64.008) (end 86.24 67.43) (width 0.25) (layer F.Cu) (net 7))
 (segment (start 86.24 67.43) (end 86.24 69.85) (width 0.25) (layer F.Cu) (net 7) (status 800000))
 (segment (start 96.012 65.194) (end 90 65.194) (width 0.25) (layer F.Cu) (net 8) (status 400000))
 (segment (start 87.74 67.454) (end 87.74 69.85) (width 0.25) (layer F.Cu) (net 8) (status 800000))
 (segment (start 90 65.194) (end 87.74 67.454) (width 0.25) (layer F.Cu) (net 8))
 (segment (start 107.315 52.07) (end 107.315 56.72) (width 0.25) (layer F.Cu) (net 9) (status 400000))
 (segment (start 107.315 56.72) (end 105.075 58.96) (width 0.25) (layer F.Cu) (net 9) (status 800000))
 (segment (start 105.075 58.96) (end 110.825 58.96) (width 0.25) (layer F.Cu) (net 9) (status 30))
 (segment (start 103.97 66.294) (end 106.088 66.294) (width 0.25) (layer F.Cu) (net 14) (status 10))
 (segment (start 130.81 55.88) (end 132.715 55.88) (width 0.25) (layer F.Cu) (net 19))
 (segment (start 134.62 53.975) (end 139.87 53.975) (width 0.25) (layer F.Cu) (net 19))
 (segment (start 132.715 55.88) (end 134.62 53.975) (width 0.25) (layer F.Cu) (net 19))
 (segment (start 130.81 52.07) (end 133.985 52.07) (width 0.25) (layer F.Cu) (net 20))
 (segment (start 134.62 51.435) (end 139.87 51.435) (width 0.25) (layer F.Cu) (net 20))
 (segment (start 133.985 52.07) (end 134.62 51.435) (width 0.25) (layer F.Cu) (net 20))
 (segment (start 122.82678 59.69) (end 125.095 59.69) (width 0.25) (layer F.Cu) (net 21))
 (segment (start 133.985 59.69) (end 125.095 59.69) (width 0.25) (layer B.Cu) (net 21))
 (segment (start 135.72 66.505) (end 136.525 66.505) (width 0.25) (layer F.Cu) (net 21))
 (via (at 135.255 60.96) (size 0.6858) (drill 0.3302) (layers F.Cu B.Cu) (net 21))
 (via (at 125.095 59.69) (size 0.6858) (drill 0.3302) (layers F.Cu B.Cu) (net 21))
 (segment (start 135.255 66.04) (end 135.255 60.96) (width 0.25) (layer F.Cu) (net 21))
 (segment (start 135.72 66.505) (end 135.255 66.04) (width 0.25) (layer F.Cu) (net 21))
 (segment (start 135.255 60.96) (end 133.985 59.69) (width 0.25) (layer B.Cu) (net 21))
 (segment (start 122.82678 59.69) (end 122.555 59.41822) (width 0.25) (layer F.Cu) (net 21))
 (segment (start 135.89 69.85) (end 135.89 68.58) (width 0.25) (layer F.Cu) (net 21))
 (segment (start 135.89 68.58) (end 136.525 67.945) (width 0.25) (layer F.Cu) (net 21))
 (segment (start 136.525 67.945) (end 136.525 66.505) (width 0.25) (layer F.Cu) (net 21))
 (segment (start 130.97 65.405) (end 133.35 65.405) (width 0.5) (layer F.Cu) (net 22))
 (segment (start 130.97 64.135) (end 133.35 64.135) (width 0.5) (layer F.Cu) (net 22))
 (segment (start 130.97 62.865) (end 133.35 62.865) (width 0.5) (layer F.Cu) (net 22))
 (segment (start 130.97 61.595) (end 132.715 61.595) (width 0.5) (layer F.Cu) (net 22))
 (segment (start 133.35 62.23) (end 133.35 62.865) (width 1.36) (layer F.Cu) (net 22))
 (segment (start 133.35 62.865) (end 133.35 64.135) (width 1.36) (layer F.Cu) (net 22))
 (segment (start 133.35 64.135) (end 133.35 65.405) (width 1.36) (layer F.Cu) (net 22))
 (segment (start 133.35 65.405) (end 133.35 69.85) (width 1.36) (layer F.Cu) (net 22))
 (segment (start 132.715 61.595) (end 133.35 62.23) (width 0.5) (layer F.Cu) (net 22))
 (segment (start 108.288 66.294) (end 110.744 66.294) (width 0.25) (layer F.Cu) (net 23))
 (segment (start 110.744 66.294) (end 111.76 67.31) (width 0.25) (layer F.Cu) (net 23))
 (segment (start 123.19 65.235) (end 123.909 65.235) (width 0.25) (layer F.Cu) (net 24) (status 400000))
 (segment (start 124.079 65.405) (end 125.57 65.405) (width 0.25) (layer F.Cu) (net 24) (status 800000))
 (segment (start 123.909 65.235) (end 124.079 65.405) (width 0.25) (layer F.Cu) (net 24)))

